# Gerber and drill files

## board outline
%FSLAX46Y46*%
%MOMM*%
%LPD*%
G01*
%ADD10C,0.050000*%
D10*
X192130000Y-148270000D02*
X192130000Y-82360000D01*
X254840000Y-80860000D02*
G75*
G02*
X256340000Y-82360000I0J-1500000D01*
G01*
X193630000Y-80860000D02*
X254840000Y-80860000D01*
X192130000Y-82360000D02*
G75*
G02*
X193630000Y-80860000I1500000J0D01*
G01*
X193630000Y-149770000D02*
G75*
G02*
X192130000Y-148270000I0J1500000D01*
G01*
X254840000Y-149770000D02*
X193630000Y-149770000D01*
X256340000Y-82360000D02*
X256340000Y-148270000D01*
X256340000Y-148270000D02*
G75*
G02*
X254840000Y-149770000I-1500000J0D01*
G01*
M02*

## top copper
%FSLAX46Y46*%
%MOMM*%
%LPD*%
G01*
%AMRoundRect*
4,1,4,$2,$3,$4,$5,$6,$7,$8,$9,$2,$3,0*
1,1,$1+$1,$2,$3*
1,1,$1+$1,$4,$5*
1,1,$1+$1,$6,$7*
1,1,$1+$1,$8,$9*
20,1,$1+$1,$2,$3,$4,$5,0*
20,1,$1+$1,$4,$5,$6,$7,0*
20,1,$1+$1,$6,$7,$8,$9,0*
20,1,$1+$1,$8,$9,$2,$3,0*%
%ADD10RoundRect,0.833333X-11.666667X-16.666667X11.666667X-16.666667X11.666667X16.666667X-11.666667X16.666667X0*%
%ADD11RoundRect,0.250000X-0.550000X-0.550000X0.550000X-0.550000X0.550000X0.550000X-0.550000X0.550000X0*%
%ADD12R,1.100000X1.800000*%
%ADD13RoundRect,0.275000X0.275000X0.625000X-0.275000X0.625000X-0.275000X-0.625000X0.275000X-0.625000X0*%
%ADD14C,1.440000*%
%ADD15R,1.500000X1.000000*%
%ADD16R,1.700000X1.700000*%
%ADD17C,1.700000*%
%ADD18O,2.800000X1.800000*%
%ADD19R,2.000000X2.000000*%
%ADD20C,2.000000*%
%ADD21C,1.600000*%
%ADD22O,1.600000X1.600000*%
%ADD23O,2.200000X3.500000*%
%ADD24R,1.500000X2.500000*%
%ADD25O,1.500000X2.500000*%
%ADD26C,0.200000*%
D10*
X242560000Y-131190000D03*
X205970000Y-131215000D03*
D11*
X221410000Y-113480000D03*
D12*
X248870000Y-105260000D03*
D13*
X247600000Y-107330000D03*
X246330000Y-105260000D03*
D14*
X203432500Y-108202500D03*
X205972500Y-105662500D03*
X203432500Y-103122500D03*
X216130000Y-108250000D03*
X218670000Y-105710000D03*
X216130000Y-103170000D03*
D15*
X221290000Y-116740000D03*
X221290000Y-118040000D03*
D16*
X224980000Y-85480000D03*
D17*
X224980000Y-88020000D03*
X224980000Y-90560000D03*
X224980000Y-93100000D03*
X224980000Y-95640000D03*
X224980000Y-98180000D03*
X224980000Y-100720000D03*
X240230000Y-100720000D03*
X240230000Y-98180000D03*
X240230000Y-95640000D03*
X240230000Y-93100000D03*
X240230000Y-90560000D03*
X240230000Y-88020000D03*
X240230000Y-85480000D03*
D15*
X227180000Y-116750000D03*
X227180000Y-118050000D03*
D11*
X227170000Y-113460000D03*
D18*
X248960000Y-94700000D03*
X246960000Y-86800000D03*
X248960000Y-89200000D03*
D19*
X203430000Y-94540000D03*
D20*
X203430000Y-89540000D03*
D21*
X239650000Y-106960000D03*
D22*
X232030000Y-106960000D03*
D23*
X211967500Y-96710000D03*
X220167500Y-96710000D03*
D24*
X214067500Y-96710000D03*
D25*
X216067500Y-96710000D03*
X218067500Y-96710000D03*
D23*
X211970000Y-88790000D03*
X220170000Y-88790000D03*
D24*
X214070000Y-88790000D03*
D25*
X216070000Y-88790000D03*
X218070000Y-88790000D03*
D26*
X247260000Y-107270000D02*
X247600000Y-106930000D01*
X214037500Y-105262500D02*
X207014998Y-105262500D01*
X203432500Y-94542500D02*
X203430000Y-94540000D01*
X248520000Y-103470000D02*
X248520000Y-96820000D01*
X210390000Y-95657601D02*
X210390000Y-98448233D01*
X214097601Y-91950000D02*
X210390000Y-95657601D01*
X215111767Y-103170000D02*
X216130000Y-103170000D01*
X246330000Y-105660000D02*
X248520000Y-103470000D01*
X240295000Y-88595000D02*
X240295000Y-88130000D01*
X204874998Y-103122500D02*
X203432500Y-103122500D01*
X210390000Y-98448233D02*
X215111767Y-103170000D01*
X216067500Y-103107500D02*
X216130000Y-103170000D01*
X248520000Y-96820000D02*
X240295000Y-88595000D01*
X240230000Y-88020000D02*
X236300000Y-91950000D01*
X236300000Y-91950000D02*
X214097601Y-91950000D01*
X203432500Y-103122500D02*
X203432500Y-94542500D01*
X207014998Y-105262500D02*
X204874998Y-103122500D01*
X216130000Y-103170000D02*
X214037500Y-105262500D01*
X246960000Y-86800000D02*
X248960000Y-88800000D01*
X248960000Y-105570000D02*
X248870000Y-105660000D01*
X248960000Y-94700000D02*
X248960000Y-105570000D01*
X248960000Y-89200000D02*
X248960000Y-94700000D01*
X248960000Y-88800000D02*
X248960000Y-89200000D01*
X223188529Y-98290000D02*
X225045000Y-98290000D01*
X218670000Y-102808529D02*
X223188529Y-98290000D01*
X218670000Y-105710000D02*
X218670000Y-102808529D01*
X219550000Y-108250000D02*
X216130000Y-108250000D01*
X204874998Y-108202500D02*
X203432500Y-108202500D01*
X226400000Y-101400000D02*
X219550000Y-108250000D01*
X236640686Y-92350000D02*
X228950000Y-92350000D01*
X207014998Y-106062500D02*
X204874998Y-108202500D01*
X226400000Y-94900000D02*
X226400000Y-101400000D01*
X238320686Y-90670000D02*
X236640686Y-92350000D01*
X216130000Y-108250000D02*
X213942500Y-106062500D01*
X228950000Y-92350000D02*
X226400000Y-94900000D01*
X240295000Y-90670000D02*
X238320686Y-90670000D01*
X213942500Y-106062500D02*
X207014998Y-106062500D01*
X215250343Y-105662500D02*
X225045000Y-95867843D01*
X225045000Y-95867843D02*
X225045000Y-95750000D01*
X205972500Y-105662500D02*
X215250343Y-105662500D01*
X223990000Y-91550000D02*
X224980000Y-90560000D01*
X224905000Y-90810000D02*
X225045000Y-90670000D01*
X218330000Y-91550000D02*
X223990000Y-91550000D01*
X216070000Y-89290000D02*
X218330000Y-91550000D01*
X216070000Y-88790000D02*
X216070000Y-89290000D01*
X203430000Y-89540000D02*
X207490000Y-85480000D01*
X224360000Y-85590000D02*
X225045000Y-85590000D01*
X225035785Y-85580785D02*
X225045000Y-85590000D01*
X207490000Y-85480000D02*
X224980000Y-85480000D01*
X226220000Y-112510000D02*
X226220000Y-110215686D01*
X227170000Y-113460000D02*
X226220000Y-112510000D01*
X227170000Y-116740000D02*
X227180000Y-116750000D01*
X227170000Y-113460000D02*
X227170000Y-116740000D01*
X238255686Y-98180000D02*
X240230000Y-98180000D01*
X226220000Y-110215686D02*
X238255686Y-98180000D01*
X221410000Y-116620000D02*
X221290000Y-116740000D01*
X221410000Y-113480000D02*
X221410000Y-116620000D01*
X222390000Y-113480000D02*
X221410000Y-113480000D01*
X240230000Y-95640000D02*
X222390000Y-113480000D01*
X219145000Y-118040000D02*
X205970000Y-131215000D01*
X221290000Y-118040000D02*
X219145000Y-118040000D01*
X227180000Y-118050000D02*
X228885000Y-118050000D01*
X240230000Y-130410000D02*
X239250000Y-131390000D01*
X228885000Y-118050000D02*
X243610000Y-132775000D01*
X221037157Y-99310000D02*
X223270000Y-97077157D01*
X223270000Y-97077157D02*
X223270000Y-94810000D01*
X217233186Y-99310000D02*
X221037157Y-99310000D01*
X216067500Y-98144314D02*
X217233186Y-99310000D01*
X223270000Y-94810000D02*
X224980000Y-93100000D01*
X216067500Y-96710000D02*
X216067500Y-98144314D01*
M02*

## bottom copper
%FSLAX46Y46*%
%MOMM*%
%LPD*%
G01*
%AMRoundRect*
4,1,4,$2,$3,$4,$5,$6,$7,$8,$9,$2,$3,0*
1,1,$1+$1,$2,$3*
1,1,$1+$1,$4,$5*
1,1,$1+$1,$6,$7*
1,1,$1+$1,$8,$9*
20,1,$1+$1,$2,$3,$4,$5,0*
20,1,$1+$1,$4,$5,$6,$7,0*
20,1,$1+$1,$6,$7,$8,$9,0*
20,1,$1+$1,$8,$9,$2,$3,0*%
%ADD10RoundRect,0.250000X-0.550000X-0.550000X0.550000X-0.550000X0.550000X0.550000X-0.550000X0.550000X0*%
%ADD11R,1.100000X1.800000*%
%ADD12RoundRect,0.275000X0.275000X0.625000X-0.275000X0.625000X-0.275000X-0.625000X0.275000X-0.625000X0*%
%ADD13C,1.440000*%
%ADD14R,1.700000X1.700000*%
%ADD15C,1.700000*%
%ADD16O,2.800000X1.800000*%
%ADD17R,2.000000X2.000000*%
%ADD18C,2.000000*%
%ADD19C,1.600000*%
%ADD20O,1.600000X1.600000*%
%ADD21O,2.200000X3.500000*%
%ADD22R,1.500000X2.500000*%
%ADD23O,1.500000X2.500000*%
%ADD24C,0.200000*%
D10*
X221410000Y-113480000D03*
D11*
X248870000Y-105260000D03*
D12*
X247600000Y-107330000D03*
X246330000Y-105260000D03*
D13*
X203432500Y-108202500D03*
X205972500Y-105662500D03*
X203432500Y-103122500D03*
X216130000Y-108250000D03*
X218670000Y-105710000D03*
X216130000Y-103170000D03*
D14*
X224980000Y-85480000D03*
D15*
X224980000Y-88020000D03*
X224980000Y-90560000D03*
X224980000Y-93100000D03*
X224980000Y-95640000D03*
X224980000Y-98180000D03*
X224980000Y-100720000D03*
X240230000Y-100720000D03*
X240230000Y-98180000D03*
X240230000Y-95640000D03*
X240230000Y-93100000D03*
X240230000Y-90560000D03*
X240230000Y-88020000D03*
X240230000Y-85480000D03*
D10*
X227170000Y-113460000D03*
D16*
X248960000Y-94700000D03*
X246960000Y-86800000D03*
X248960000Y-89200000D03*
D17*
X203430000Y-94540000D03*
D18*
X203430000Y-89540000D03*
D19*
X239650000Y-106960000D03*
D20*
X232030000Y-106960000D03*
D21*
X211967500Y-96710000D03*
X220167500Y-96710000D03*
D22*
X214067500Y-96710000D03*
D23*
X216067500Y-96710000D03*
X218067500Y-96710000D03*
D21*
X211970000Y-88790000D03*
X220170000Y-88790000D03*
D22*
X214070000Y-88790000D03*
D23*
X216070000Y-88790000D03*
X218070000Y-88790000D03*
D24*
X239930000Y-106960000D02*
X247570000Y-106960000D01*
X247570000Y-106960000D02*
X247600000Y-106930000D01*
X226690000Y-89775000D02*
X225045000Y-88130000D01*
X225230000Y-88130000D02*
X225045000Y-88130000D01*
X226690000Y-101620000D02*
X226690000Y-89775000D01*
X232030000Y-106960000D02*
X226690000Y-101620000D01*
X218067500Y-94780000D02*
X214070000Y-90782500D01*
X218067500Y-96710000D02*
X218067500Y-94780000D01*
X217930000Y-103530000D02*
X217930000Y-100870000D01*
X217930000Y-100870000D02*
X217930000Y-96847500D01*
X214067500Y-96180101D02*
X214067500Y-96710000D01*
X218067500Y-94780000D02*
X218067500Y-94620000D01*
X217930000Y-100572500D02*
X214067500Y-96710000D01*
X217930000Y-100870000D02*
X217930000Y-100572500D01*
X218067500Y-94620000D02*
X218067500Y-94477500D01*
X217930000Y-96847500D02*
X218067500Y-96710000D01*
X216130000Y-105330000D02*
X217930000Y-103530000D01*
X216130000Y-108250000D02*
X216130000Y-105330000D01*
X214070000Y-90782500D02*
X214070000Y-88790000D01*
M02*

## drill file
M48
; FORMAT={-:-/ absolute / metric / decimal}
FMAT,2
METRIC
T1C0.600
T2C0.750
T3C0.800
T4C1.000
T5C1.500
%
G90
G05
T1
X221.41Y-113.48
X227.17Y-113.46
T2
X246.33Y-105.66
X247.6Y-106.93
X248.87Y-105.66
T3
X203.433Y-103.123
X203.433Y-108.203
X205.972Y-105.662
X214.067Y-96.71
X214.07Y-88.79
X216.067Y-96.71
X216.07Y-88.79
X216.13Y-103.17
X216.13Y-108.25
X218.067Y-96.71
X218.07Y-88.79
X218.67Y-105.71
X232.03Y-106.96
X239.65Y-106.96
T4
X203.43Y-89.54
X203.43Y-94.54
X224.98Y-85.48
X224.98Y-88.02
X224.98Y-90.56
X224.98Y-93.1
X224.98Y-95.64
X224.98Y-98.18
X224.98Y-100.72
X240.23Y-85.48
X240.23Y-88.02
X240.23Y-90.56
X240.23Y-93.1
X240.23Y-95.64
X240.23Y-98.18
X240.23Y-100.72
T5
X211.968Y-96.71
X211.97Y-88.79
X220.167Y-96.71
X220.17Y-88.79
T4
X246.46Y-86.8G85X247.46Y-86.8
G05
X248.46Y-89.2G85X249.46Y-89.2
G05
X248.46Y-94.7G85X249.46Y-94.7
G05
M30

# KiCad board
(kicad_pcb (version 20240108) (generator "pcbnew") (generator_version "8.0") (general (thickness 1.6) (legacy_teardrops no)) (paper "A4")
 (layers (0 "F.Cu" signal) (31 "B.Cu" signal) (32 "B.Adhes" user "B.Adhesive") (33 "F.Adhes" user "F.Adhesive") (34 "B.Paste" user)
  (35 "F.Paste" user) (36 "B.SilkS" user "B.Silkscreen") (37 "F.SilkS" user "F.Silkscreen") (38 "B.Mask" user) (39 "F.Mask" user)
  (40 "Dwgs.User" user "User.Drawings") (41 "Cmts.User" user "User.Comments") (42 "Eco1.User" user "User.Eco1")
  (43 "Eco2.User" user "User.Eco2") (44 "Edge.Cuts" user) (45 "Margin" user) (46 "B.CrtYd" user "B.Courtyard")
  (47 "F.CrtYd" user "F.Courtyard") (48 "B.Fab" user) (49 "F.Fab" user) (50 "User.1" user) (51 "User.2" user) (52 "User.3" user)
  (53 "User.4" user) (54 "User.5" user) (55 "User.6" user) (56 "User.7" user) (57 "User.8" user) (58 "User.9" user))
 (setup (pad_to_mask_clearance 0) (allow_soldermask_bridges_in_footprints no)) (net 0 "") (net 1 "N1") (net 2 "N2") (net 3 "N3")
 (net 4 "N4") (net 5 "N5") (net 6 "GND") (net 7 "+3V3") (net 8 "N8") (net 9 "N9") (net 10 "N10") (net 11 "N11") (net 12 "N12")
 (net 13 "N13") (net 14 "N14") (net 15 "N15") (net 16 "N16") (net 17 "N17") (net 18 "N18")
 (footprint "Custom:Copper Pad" (layer "F.Cu") (at 251.06 110.19)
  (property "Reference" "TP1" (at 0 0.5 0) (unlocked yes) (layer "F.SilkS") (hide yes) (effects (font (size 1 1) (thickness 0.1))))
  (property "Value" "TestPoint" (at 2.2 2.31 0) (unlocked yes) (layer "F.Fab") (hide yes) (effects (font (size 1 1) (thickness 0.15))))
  (pad "1" smd roundrect (at -8.5 21) (size 25 35) (layers "F.Cu" "F.Mask") (roundrect_rratio 0.03333333333) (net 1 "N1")))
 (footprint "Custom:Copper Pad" (layer "F.Cu") (at 211.47 110.715)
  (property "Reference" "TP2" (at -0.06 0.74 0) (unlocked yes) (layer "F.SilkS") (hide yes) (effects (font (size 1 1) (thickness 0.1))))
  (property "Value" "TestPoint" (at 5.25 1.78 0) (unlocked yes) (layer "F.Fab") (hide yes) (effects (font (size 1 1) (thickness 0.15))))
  (pad "1" smd roundrect (at -5.5 20.5) (size 25 35) (layers "F.Cu" "F.Mask") (roundrect_rratio 0.03333333333) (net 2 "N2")))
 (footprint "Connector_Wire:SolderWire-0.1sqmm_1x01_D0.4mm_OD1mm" (layer "F.Cu") (at 221.41 113.48)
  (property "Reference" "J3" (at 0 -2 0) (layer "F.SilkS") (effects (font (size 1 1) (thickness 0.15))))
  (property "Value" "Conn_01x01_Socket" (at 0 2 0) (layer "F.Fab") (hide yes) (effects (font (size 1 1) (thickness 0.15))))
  (pad "1" thru_hole roundrect (at 0 0) (size 1.6 1.6) (drill 0.6) (layers "*.Cu" "*.Mask") (remove_unused_layers no)
   (roundrect_rratio 0.15625) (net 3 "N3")))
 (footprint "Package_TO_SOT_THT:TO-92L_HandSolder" (layer "F.Cu") (at 248.87 105.66 180)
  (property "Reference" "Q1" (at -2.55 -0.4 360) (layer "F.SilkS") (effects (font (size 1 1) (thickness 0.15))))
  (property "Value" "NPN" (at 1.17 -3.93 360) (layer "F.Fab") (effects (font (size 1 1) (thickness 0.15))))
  (pad "1" thru_hole rect (at 0 0 180) (size 1.1 1.8) (drill 0.75 (offset 0 0.4)) (layers "*.Cu" "*.Mask") (remove_unused_layers no)
   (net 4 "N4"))
  (pad "2" thru_hole roundrect (at 1.27 -1.27 180) (size 1.1 1.8) (drill 0.75 (offset 0 -0.4)) (layers "*.Cu" "*.Mask")
   (remove_unused_layers no) (roundrect_rratio 0.25) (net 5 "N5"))
  (pad "3" thru_hole roundrect (at 2.54 0 180) (size 1.1 1.8) (drill 0.75 (offset 0 0.4)) (layers "*.Cu" "*.Mask") (remove_unused_layers no)
   (roundrect_rratio 0.25) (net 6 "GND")))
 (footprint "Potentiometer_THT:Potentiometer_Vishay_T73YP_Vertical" (layer "F.Cu") (at 203.4325 108.2025)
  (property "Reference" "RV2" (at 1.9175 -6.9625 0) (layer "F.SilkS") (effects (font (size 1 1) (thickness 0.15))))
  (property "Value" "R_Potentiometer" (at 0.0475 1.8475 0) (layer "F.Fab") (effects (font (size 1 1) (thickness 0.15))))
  (pad "1" thru_hole circle (at 0 0) (size 1.44 1.44) (drill 0.8) (layers "*.Cu" "*.Mask") (remove_unused_layers no) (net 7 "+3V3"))
  (pad "2" thru_hole circle (at 2.54 -2.54) (size 1.44 1.44) (drill 0.8) (layers "*.Cu" "*.Mask") (remove_unused_layers no) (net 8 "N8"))
  (pad "3" thru_hole circle (at 0 -5.08) (size 1.44 1.44) (drill 0.8) (layers "*.Cu" "*.Mask") (remove_unused_layers no) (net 6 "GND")))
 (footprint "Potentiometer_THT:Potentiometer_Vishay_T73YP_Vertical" (layer "F.Cu") (at 216.13 108.25)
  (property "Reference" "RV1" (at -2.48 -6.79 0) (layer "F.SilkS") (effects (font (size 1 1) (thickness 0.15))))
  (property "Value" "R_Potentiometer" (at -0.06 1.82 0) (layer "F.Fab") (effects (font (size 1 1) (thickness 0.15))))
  (pad "1" thru_hole circle (at 0 0) (size 1.44 1.44) (drill 0.8) (layers "*.Cu" "*.Mask") (remove_unused_layers no) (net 7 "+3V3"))
  (pad "2" thru_hole circle (at 2.54 -2.54) (size 1.44 1.44) (drill 0.8) (layers "*.Cu" "*.Mask") (remove_unused_layers no) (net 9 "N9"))
  (pad "3" thru_hole circle (at 0 -5.08) (size 1.44 1.44) (drill 0.8) (layers "*.Cu" "*.Mask") (remove_unused_layers no) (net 6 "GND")))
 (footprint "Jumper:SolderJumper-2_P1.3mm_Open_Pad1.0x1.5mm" (layer "F.Cu") (at 221.29 117.39 -90)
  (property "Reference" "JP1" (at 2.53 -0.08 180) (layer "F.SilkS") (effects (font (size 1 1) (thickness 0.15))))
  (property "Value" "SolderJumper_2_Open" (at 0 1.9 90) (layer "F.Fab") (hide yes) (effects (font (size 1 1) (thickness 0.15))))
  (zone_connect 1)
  (pad "1" smd rect (at -0.65 0 270) (size 1 1.5) (layers "F.Cu" "F.Mask") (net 3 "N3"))
  (pad "2" smd rect (at 0.65 0 270) (size 1 1.5) (layers "F.Cu" "F.Mask") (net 2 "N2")))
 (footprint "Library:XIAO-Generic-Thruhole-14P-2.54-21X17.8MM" (layer "F.Cu") (at 232.605 93.1)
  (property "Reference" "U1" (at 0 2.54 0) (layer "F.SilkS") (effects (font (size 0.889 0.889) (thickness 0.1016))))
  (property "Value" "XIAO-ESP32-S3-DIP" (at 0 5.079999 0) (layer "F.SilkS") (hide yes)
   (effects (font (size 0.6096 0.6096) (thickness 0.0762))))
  (pad "1" thru_hole rect (at -7.625 -7.62 180) (size 1.7 1.7) (drill 1) (layers "*.Cu" "*.Mask") (remove_unused_layers no) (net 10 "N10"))
  (pad "2" thru_hole circle (at -7.625 -5.08 180) (size 1.7 1.7) (drill 1) (layers "*.Cu" "*.Mask") (remove_unused_layers no) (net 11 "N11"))
  (pad "3" thru_hole circle (at -7.625 -2.54 180) (size 1.7 1.7) (drill 1) (layers "*.Cu" "*.Mask") (remove_unused_layers no) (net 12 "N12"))
  (pad "4" thru_hole circle (at -7.625 0 180) (size 1.7 1.7) (drill 1) (layers "*.Cu" "*.Mask") (remove_unused_layers no) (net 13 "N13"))
  (pad "5" thru_hole circle (at -7.625 2.54 180) (size 1.7 1.7) (drill 1) (layers "*.Cu" "*.Mask") (remove_unused_layers no) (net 8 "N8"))
  (pad "6" thru_hole circle (at -7.625 5.08) (size 1.7 1.7) (drill 1) (layers "*.Cu" "*.Mask") (remove_unused_layers no) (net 9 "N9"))
  (pad "7" thru_hole circle (at -7.625 7.62 180) (size 1.7 1.7) (drill 1) (layers "*.Cu" "*.Mask") (remove_unused_layers no) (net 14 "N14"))
  (pad "8" thru_hole circle (at 7.625 7.62 180) (size 1.7 1.7) (drill 1) (layers "*.Cu" "*.Mask") (remove_unused_layers no) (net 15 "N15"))
  (pad "9" thru_hole circle (at 7.625 5.08 180) (size 1.7 1.7) (drill 1) (layers "*.Cu" "*.Mask") (remove_unused_layers no) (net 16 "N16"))
  (pad "10" thru_hole circle (at 7.625 2.54 180) (size 1.7 1.7) (drill 1) (layers "*.Cu" "*.Mask") (remove_unused_layers no) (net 3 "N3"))
  (pad "11" thru_hole circle (at 7.625 0 180) (size 1.7 1.7) (drill 1) (layers "*.Cu" "*.Mask") (remove_unused_layers no) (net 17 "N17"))
  (pad "12" thru_hole circle (at 7.625 -2.54 180) (size 1.7 1.7) (drill 1) (layers "*.Cu" "*.Mask") (remove_unused_layers no) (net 7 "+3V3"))
  (pad "13" thru_hole circle (at 7.625 -5.08 180) (size 1.7 1.7) (drill 1) (layers "*.Cu" "*.Mask") (remove_unused_layers no) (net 6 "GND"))
  (pad "14" thru_hole circle (at 7.625 -7.62 180) (size 1.7 1.7) (drill 1) (layers "*.Cu" "*.Mask") (remove_unused_layers no) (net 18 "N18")))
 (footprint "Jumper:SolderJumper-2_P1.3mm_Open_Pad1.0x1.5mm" (layer "F.Cu") (at 227.18 117.4 -90)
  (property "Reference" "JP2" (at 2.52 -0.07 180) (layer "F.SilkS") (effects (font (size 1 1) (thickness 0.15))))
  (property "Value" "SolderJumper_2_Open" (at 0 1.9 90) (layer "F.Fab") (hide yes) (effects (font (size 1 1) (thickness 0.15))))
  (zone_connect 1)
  (pad "1" smd rect (at -0.65 0 270) (size 1 1.5) (layers "F.Cu" "F.Mask") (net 16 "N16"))
  (pad "2" smd rect (at 0.65 0 270) (size 1 1.5) (layers "F.Cu" "F.Mask") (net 1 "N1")))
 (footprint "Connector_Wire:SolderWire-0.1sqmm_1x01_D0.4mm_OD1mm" (layer "F.Cu") (at 227.17 113.46)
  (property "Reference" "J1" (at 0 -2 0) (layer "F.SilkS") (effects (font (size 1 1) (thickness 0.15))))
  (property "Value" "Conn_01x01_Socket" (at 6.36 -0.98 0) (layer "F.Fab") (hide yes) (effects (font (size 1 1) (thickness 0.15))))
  (pad "1" thru_hole roundrect (at 0 0) (size 1.6 1.6) (drill 0.6) (layers "*.Cu" "*.Mask") (remove_unused_layers no)
   (roundrect_rratio 0.15625) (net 16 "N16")))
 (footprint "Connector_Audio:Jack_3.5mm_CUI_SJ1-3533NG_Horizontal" (layer "F.Cu") (at 246.96 86.8)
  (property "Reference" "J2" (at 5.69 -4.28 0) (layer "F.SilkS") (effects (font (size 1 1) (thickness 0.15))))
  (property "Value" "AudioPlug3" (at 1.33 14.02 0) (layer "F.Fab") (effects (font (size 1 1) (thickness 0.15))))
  (pad "R" thru_hole oval (at 2 7.9) (size 2.8 1.8) (drill oval 2 1) (layers "*.Cu" "*.Mask") (remove_unused_layers no) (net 4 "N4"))
  (pad "S" thru_hole oval (at 0 0) (size 2.8 1.8) (drill oval 2 1) (layers "*.Cu" "*.Mask") (remove_unused_layers no) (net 4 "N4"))
  (pad "T" thru_hole oval (at 2 2.4) (size 2.8 1.8) (drill oval 2 1) (layers "*.Cu" "*.Mask") (remove_unused_layers no) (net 4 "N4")))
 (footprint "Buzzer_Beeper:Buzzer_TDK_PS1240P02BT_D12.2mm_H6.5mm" (layer "F.Cu") (at 203.43 94.54 90)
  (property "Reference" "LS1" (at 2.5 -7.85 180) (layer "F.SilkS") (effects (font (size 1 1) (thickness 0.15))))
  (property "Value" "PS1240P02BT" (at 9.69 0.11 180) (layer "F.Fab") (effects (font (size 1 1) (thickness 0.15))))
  (pad "1" thru_hole rect (at 0 0 90) (size 2 2) (drill 1) (layers "*.Cu" "*.Mask") (remove_unused_layers no) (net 6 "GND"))
  (pad "2" thru_hole circle (at 5 0 90) (size 2 2) (drill 1) (layers "*.Cu" "*.Mask") (remove_unused_layers no) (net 10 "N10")))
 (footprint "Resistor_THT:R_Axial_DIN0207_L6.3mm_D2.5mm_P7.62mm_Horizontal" (layer "F.Cu") (at 239.65 106.96 180)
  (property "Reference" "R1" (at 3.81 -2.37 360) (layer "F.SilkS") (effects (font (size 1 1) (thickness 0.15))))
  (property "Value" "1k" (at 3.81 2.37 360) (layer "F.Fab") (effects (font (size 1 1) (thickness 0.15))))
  (pad "1" thru_hole circle (at 0 0 180) (size 1.6 1.6) (drill 0.8) (layers "*.Cu" "*.Mask") (remove_unused_layers no) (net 5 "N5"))
  (pad "2" thru_hole oval (at 7.62 0 180) (size 1.6 1.6) (drill 0.8) (layers "*.Cu" "*.Mask") (remove_unused_layers no) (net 11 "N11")))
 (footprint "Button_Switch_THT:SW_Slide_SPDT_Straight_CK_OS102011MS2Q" (layer "F.Cu") (at 214.0675 96.71)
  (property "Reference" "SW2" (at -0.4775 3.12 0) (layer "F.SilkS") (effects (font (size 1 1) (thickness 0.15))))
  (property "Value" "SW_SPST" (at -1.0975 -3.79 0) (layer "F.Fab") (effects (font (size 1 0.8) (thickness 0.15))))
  (pad "" thru_hole oval (at -2.1 0) (size 2.2 3.5) (drill 1.5) (layers "*.Cu" "*.Mask") (remove_unused_layers no))
  (pad "" thru_hole oval (at 6.1 0) (size 2.2 3.5) (drill 1.5) (layers "*.Cu" "*.Mask") (remove_unused_layers no))
  (pad "1" thru_hole rect (at 0 0) (size 1.5 2.5) (drill 0.8) (layers "*.Cu" "*.Mask") (remove_unused_layers no) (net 7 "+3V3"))
  (pad "2" thru_hole oval (at 2 0) (size 1.5 2.5) (drill 0.8) (layers "*.Cu" "*.Mask") (remove_unused_layers no) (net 13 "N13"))
  (pad "3" thru_hole oval (at 4 0) (size 1.5 2.5) (drill 0.8) (layers "*.Cu" "*.Mask") (remove_unused_layers no)))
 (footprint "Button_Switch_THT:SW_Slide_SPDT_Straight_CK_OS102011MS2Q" (layer "F.Cu") (at 214.07 88.79)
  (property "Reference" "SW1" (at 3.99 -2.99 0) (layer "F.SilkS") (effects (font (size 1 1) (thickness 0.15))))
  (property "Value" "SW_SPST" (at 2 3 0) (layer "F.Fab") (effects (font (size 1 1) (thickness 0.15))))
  (pad "" thru_hole oval (at -2.1 0) (size 2.2 3.5) (drill 1.5) (layers "*.Cu" "*.Mask") (remove_unused_layers no))
  (pad "" thru_hole oval (at 6.1 0) (size 2.2 3.5) (drill 1.5) (layers "*.Cu" "*.Mask") (remove_unused_layers no))
  (pad "1" thru_hole rect (at 0 0) (size 1.5 2.5) (drill 0.8) (layers "*.Cu" "*.Mask") (remove_unused_layers no) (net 7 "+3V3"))
  (pad "2" thru_hole oval (at 2 0) (size 1.5 2.5) (drill 0.8) (layers "*.Cu" "*.Mask") (remove_unused_layers no) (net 12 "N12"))
  (pad "3" thru_hole oval (at 4 0) (size 1.5 2.5) (drill 0.8) (layers "*.Cu" "*.Mask") (remove_unused_layers no)))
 (gr_line (start 192.13 148.27) (end 192.13 82.36) (stroke (width 0.05) (type default)) (layer "Edge.Cuts"))
 (gr_arc (start 254.84 80.86) (mid 255.90066 81.29934) (end 256.34 82.36) (stroke (width 0.05) (type default)) (layer "Edge.Cuts"))
 (gr_line (start 193.63 80.86) (end 254.84 80.86) (stroke (width 0.05) (type default)) (layer "Edge.Cuts"))
 (gr_arc (start 192.13 82.36) (mid 192.56934 81.29934) (end 193.63 80.86) (stroke (width 0.05) (type default)) (layer "Edge.Cuts"))
 (gr_arc (start 193.63 149.77) (mid 192.56934 149.33066) (end 192.13 148.27) (stroke (width 0.05) (type default)) (layer "Edge.Cuts"))
 (gr_line (start 254.84 149.77) (end 193.63 149.77) (stroke (width 0.05) (type default)) (layer "Edge.Cuts"))
 (gr_line (start 256.34 82.36) (end 256.34 148.27) (stroke (width 0.05) (type default)) (layer "Edge.Cuts"))
 (gr_arc (start 256.34 148.27) (mid 255.90066 149.33066) (end 254.84 149.77) (stroke (width 0.05) (type default)) (layer "Edge.Cuts"))
 (segment (start 247.26 107.27) (end 247.6 106.93) (width 0.2) (layer "F.Cu") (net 5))
 (segment (start 239.93 106.96) (end 247.57 106.96) (width 0.2) (layer "B.Cu") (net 5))
 (segment (start 247.57 106.96) (end 247.6 106.93) (width 0.2) (layer "B.Cu") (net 5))
 (segment (start 214.0375 105.2625) (end 207.014998 105.2625) (width 0.2) (layer "F.Cu") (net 6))
 (segment (start 203.4325 94.5425) (end 203.43 94.54) (width 0.2) (layer "F.Cu") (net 6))
 (segment (start 248.52 103.47) (end 248.52 96.82) (width 0.2) (layer "F.Cu") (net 6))
 (segment (start 210.39 95.657601) (end 210.39 98.448233) (width 0.2) (layer "F.Cu") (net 6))
 (segment (start 214.097601 91.95) (end 210.39 95.657601) (width 0.2) (layer "F.Cu") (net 6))
 (segment (start 215.111767 103.17) (end 216.13 103.17) (width 0.2) (layer "F.Cu") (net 6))
 (segment (start 246.33 105.66) (end 248.52 103.47) (width 0.2) (layer "F.Cu") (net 6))
 (segment (start 240.295 88.595) (end 240.295 88.13) (width 0.2) (layer "F.Cu") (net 6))
 (segment (start 204.874998 103.1225) (end 203.4325 103.1225) (width 0.2) (layer "F.Cu") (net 6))
 (segment (start 210.39 98.448233) (end 215.111767 103.17) (width 0.2) (layer "F.Cu") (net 6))
 (segment (start 216.0675 103.1075) (end 216.13 103.17) (width 0.2) (layer "F.Cu") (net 6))
 (segment (start 248.52 96.82) (end 240.295 88.595) (width 0.2) (layer "F.Cu") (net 6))
 (segment (start 240.23 88.02) (end 236.3 91.95) (width 0.2) (layer "F.Cu") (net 6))
 (segment (start 236.3 91.95) (end 214.097601 91.95) (width 0.2) (layer "F.Cu") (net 6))
 (segment (start 203.4325 103.1225) (end 203.4325 94.5425) (width 0.2) (layer "F.Cu") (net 6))
 (segment (start 207.014998 105.2625) (end 204.874998 103.1225) (width 0.2) (layer "F.Cu") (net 6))
 (segment (start 216.13 103.17) (end 214.0375 105.2625) (width 0.2) (layer "F.Cu") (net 6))
 (segment (start 246.96 86.8) (end 248.96 88.8) (width 0.2) (layer "F.Cu") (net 4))
 (segment (start 248.96 105.57) (end 248.87 105.66) (width 0.2) (layer "F.Cu") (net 4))
 (segment (start 248.96 94.7) (end 248.96 105.57) (width 0.2) (layer "F.Cu") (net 4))
 (segment (start 248.96 89.2) (end 248.96 94.7) (width 0.2) (layer "F.Cu") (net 4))
 (segment (start 248.96 88.8) (end 248.96 89.2) (width 0.2) (layer "F.Cu") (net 4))
 (segment (start 226.69 89.775) (end 225.045 88.13) (width 0.2) (layer "B.Cu") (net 11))
 (segment (start 225.23 88.13) (end 225.045 88.13) (width 0.2) (layer "B.Cu") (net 11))
 (segment (start 226.69 101.62) (end 226.69 89.775) (width 0.2) (layer "B.Cu") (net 11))
 (segment (start 232.03 106.96) (end 226.69 101.62) (width 0.2) (layer "B.Cu") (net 11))
 (segment (start 223.188529 98.29) (end 225.045 98.29) (width 0.2) (layer "F.Cu") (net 9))
 (segment (start 218.67 102.808529) (end 223.188529 98.29) (width 0.2) (layer "F.Cu") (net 9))
 (segment (start 218.67 105.71) (end 218.67 102.808529) (width 0.2) (layer "F.Cu") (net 9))
 (segment (start 219.55 108.25) (end 216.13 108.25) (width 0.2) (layer "F.Cu") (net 7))
 (segment (start 204.874998 108.2025) (end 203.4325 108.2025) (width 0.2) (layer "F.Cu") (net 7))
 (segment (start 226.4 101.4) (end 219.55 108.25) (width 0.2) (layer "F.Cu") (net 7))
 (segment (start 236.640686 92.35) (end 228.95 92.35) (width 0.2) (layer "F.Cu") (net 7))
 (segment (start 207.014998 106.0625) (end 204.874998 108.2025) (width 0.2) (layer "F.Cu") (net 7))
 (segment (start 226.4 94.9) (end 226.4 101.4) (width 0.2) (layer "F.Cu") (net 7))
 (segment (start 238.320686 90.67) (end 236.640686 92.35) (width 0.2) (layer "F.Cu") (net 7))
 (segment (start 216.13 108.25) (end 213.9425 106.0625) (width 0.2) (layer "F.Cu") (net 7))
 (segment (start 228.95 92.35) (end 226.4 94.9) (width 0.2) (layer "F.Cu") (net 7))
 (segment (start 240.295 90.67) (end 238.320686 90.67) (width 0.2) (layer "F.Cu") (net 7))
 (segment (start 213.9425 106.0625) (end 207.014998 106.0625) (width 0.2) (layer "F.Cu") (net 7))
 (segment (start 218.0675 94.78) (end 214.07 90.7825) (width 0.2) (layer "B.Cu") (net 7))
 (segment (start 218.0675 96.71) (end 218.0675 94.78) (width 0.2) (layer "B.Cu") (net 7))
 (segment (start 217.93 103.53) (end 217.93 100.87) (width 0.2) (layer "B.Cu") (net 7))
 (segment (start 217.93 100.87) (end 217.93 96.8475) (width 0.2) (layer "B.Cu") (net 7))
 (segment (start 214.0675 96.180101) (end 214.0675 96.71) (width 0.2) (layer "B.Cu") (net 7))
 (segment (start 218.0675 94.78) (end 218.0675 94.62) (width 0.2) (layer "B.Cu") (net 7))
 (segment (start 217.93 100.5725) (end 214.0675 96.71) (width 0.2) (layer "B.Cu") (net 7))
 (segment (start 217.93 100.87) (end 217.93 100.5725) (width 0.2) (layer "B.Cu") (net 7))
 (segment (start 218.0675 94.62) (end 218.0675 94.4775) (width 0.2) (layer "B.Cu") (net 7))
 (segment (start 217.93 96.8475) (end 218.0675 96.71) (width 0.2) (layer "B.Cu") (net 7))
 (segment (start 216.13 105.33) (end 217.93 103.53) (width 0.2) (layer "B.Cu") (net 7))
 (segment (start 216.13 108.25) (end 216.13 105.33) (width 0.2) (layer "B.Cu") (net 7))
 (segment (start 214.07 90.7825) (end 214.07 88.79) (width 0.2) (layer "B.Cu") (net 7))
 (segment (start 215.250343 105.6625) (end 225.045 95.867843) (width 0.2) (layer "F.Cu") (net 8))
 (segment (start 225.045 95.867843) (end 225.045 95.75) (width 0.2) (layer "F.Cu") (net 8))
 (segment (start 205.9725 105.6625) (end 215.250343 105.6625) (width 0.2) (layer "F.Cu") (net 8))
 (segment (start 223.99 91.55) (end 224.98 90.56) (width 0.2) (layer "F.Cu") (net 12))
 (segment (start 224.905 90.81) (end 225.045 90.67) (width 0.2) (layer "F.Cu") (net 12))
 (segment (start 218.33 91.55) (end 223.99 91.55) (width 0.2) (layer "F.Cu") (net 12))
 (segment (start 216.07 89.29) (end 218.33 91.55) (width 0.2) (layer "F.Cu") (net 12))
 (segment (start 216.07 88.79) (end 216.07 89.29) (width 0.2) (layer "F.Cu") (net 12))
 (segment (start 203.43 89.54) (end 207.49 85.48) (width 0.2) (layer "F.Cu") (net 10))
 (segment (start 224.36 85.59) (end 225.045 85.59) (width 0.2) (layer "F.Cu") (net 10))
 (segment (start 225.035785 85.580785) (end 225.045 85.59) (width 0.2) (layer "F.Cu") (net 10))
 (segment (start 207.49 85.48) (end 224.98 85.48) (width 0.2) (layer "F.Cu") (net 10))
 (segment (start 226.22 112.51) (end 226.22 110.215686) (width 0.2) (layer "F.Cu") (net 16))
 (segment (start 227.17 113.46) (end 226.22 112.51) (width 0.2) (layer "F.Cu") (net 16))
 (segment (start 227.17 116.74) (end 227.18 116.75) (width 0.2) (layer "F.Cu") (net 16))
 (segment (start 227.17 113.46) (end 227.17 116.74) (width 0.2) (layer "F.Cu") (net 16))
 (segment (start 238.255686 98.18) (end 240.23 98.18) (width 0.2) (layer "F.Cu") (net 16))
 (segment (start 226.22 110.215686) (end 238.255686 98.18) (width 0.2) (layer "F.Cu") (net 16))
 (segment (start 221.41 116.62) (end 221.29 116.74) (width 0.2) (layer "F.Cu") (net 3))
 (segment (start 221.41 113.48) (end 221.41 116.62) (width 0.2) (layer "F.Cu") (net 3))
 (segment (start 222.39 113.48) (end 221.41 113.48) (width 0.2) (layer "F.Cu") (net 3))
 (segment (start 240.23 95.64) (end 222.39 113.48) (width 0.2) (layer "F.Cu") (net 3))
 (segment (start 219.145 118.04) (end 205.97 131.215) (width 0.2) (layer "F.Cu") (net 2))
 (segment (start 221.29 118.04) (end 219.145 118.04) (width 0.2) (layer "F.Cu") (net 2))
 (segment (start 227.18 118.05) (end 228.885 118.05) (width 0.2) (layer "F.Cu") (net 1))
 (segment (start 240.23 130.41) (end 239.25 131.39) (width 0.2) (layer "F.Cu") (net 1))
 (segment (start 228.885 118.05) (end 243.61 132.775) (width 0.2) (layer "F.Cu") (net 1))
 (segment (start 221.037157 99.31) (end 223.27 97.077157) (width 0.2) (layer "F.Cu") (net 13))
 (segment (start 223.27 97.077157) (end 223.27 94.81) (width 0.2) (layer "F.Cu") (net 13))
 (segment (start 217.233186 99.31) (end 221.037157 99.31) (width 0.2) (layer "F.Cu") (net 13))
 (segment (start 216.0675 98.144314) (end 217.233186 99.31) (width 0.2) (layer "F.Cu") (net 13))
 (segment (start 223.27 94.81) (end 224.98 93.1) (width 0.2) (layer "F.Cu") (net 13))
 (segment (start 216.0675 96.71) (end 216.0675 98.144314) (width 0.2) (layer "F.Cu") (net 13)))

